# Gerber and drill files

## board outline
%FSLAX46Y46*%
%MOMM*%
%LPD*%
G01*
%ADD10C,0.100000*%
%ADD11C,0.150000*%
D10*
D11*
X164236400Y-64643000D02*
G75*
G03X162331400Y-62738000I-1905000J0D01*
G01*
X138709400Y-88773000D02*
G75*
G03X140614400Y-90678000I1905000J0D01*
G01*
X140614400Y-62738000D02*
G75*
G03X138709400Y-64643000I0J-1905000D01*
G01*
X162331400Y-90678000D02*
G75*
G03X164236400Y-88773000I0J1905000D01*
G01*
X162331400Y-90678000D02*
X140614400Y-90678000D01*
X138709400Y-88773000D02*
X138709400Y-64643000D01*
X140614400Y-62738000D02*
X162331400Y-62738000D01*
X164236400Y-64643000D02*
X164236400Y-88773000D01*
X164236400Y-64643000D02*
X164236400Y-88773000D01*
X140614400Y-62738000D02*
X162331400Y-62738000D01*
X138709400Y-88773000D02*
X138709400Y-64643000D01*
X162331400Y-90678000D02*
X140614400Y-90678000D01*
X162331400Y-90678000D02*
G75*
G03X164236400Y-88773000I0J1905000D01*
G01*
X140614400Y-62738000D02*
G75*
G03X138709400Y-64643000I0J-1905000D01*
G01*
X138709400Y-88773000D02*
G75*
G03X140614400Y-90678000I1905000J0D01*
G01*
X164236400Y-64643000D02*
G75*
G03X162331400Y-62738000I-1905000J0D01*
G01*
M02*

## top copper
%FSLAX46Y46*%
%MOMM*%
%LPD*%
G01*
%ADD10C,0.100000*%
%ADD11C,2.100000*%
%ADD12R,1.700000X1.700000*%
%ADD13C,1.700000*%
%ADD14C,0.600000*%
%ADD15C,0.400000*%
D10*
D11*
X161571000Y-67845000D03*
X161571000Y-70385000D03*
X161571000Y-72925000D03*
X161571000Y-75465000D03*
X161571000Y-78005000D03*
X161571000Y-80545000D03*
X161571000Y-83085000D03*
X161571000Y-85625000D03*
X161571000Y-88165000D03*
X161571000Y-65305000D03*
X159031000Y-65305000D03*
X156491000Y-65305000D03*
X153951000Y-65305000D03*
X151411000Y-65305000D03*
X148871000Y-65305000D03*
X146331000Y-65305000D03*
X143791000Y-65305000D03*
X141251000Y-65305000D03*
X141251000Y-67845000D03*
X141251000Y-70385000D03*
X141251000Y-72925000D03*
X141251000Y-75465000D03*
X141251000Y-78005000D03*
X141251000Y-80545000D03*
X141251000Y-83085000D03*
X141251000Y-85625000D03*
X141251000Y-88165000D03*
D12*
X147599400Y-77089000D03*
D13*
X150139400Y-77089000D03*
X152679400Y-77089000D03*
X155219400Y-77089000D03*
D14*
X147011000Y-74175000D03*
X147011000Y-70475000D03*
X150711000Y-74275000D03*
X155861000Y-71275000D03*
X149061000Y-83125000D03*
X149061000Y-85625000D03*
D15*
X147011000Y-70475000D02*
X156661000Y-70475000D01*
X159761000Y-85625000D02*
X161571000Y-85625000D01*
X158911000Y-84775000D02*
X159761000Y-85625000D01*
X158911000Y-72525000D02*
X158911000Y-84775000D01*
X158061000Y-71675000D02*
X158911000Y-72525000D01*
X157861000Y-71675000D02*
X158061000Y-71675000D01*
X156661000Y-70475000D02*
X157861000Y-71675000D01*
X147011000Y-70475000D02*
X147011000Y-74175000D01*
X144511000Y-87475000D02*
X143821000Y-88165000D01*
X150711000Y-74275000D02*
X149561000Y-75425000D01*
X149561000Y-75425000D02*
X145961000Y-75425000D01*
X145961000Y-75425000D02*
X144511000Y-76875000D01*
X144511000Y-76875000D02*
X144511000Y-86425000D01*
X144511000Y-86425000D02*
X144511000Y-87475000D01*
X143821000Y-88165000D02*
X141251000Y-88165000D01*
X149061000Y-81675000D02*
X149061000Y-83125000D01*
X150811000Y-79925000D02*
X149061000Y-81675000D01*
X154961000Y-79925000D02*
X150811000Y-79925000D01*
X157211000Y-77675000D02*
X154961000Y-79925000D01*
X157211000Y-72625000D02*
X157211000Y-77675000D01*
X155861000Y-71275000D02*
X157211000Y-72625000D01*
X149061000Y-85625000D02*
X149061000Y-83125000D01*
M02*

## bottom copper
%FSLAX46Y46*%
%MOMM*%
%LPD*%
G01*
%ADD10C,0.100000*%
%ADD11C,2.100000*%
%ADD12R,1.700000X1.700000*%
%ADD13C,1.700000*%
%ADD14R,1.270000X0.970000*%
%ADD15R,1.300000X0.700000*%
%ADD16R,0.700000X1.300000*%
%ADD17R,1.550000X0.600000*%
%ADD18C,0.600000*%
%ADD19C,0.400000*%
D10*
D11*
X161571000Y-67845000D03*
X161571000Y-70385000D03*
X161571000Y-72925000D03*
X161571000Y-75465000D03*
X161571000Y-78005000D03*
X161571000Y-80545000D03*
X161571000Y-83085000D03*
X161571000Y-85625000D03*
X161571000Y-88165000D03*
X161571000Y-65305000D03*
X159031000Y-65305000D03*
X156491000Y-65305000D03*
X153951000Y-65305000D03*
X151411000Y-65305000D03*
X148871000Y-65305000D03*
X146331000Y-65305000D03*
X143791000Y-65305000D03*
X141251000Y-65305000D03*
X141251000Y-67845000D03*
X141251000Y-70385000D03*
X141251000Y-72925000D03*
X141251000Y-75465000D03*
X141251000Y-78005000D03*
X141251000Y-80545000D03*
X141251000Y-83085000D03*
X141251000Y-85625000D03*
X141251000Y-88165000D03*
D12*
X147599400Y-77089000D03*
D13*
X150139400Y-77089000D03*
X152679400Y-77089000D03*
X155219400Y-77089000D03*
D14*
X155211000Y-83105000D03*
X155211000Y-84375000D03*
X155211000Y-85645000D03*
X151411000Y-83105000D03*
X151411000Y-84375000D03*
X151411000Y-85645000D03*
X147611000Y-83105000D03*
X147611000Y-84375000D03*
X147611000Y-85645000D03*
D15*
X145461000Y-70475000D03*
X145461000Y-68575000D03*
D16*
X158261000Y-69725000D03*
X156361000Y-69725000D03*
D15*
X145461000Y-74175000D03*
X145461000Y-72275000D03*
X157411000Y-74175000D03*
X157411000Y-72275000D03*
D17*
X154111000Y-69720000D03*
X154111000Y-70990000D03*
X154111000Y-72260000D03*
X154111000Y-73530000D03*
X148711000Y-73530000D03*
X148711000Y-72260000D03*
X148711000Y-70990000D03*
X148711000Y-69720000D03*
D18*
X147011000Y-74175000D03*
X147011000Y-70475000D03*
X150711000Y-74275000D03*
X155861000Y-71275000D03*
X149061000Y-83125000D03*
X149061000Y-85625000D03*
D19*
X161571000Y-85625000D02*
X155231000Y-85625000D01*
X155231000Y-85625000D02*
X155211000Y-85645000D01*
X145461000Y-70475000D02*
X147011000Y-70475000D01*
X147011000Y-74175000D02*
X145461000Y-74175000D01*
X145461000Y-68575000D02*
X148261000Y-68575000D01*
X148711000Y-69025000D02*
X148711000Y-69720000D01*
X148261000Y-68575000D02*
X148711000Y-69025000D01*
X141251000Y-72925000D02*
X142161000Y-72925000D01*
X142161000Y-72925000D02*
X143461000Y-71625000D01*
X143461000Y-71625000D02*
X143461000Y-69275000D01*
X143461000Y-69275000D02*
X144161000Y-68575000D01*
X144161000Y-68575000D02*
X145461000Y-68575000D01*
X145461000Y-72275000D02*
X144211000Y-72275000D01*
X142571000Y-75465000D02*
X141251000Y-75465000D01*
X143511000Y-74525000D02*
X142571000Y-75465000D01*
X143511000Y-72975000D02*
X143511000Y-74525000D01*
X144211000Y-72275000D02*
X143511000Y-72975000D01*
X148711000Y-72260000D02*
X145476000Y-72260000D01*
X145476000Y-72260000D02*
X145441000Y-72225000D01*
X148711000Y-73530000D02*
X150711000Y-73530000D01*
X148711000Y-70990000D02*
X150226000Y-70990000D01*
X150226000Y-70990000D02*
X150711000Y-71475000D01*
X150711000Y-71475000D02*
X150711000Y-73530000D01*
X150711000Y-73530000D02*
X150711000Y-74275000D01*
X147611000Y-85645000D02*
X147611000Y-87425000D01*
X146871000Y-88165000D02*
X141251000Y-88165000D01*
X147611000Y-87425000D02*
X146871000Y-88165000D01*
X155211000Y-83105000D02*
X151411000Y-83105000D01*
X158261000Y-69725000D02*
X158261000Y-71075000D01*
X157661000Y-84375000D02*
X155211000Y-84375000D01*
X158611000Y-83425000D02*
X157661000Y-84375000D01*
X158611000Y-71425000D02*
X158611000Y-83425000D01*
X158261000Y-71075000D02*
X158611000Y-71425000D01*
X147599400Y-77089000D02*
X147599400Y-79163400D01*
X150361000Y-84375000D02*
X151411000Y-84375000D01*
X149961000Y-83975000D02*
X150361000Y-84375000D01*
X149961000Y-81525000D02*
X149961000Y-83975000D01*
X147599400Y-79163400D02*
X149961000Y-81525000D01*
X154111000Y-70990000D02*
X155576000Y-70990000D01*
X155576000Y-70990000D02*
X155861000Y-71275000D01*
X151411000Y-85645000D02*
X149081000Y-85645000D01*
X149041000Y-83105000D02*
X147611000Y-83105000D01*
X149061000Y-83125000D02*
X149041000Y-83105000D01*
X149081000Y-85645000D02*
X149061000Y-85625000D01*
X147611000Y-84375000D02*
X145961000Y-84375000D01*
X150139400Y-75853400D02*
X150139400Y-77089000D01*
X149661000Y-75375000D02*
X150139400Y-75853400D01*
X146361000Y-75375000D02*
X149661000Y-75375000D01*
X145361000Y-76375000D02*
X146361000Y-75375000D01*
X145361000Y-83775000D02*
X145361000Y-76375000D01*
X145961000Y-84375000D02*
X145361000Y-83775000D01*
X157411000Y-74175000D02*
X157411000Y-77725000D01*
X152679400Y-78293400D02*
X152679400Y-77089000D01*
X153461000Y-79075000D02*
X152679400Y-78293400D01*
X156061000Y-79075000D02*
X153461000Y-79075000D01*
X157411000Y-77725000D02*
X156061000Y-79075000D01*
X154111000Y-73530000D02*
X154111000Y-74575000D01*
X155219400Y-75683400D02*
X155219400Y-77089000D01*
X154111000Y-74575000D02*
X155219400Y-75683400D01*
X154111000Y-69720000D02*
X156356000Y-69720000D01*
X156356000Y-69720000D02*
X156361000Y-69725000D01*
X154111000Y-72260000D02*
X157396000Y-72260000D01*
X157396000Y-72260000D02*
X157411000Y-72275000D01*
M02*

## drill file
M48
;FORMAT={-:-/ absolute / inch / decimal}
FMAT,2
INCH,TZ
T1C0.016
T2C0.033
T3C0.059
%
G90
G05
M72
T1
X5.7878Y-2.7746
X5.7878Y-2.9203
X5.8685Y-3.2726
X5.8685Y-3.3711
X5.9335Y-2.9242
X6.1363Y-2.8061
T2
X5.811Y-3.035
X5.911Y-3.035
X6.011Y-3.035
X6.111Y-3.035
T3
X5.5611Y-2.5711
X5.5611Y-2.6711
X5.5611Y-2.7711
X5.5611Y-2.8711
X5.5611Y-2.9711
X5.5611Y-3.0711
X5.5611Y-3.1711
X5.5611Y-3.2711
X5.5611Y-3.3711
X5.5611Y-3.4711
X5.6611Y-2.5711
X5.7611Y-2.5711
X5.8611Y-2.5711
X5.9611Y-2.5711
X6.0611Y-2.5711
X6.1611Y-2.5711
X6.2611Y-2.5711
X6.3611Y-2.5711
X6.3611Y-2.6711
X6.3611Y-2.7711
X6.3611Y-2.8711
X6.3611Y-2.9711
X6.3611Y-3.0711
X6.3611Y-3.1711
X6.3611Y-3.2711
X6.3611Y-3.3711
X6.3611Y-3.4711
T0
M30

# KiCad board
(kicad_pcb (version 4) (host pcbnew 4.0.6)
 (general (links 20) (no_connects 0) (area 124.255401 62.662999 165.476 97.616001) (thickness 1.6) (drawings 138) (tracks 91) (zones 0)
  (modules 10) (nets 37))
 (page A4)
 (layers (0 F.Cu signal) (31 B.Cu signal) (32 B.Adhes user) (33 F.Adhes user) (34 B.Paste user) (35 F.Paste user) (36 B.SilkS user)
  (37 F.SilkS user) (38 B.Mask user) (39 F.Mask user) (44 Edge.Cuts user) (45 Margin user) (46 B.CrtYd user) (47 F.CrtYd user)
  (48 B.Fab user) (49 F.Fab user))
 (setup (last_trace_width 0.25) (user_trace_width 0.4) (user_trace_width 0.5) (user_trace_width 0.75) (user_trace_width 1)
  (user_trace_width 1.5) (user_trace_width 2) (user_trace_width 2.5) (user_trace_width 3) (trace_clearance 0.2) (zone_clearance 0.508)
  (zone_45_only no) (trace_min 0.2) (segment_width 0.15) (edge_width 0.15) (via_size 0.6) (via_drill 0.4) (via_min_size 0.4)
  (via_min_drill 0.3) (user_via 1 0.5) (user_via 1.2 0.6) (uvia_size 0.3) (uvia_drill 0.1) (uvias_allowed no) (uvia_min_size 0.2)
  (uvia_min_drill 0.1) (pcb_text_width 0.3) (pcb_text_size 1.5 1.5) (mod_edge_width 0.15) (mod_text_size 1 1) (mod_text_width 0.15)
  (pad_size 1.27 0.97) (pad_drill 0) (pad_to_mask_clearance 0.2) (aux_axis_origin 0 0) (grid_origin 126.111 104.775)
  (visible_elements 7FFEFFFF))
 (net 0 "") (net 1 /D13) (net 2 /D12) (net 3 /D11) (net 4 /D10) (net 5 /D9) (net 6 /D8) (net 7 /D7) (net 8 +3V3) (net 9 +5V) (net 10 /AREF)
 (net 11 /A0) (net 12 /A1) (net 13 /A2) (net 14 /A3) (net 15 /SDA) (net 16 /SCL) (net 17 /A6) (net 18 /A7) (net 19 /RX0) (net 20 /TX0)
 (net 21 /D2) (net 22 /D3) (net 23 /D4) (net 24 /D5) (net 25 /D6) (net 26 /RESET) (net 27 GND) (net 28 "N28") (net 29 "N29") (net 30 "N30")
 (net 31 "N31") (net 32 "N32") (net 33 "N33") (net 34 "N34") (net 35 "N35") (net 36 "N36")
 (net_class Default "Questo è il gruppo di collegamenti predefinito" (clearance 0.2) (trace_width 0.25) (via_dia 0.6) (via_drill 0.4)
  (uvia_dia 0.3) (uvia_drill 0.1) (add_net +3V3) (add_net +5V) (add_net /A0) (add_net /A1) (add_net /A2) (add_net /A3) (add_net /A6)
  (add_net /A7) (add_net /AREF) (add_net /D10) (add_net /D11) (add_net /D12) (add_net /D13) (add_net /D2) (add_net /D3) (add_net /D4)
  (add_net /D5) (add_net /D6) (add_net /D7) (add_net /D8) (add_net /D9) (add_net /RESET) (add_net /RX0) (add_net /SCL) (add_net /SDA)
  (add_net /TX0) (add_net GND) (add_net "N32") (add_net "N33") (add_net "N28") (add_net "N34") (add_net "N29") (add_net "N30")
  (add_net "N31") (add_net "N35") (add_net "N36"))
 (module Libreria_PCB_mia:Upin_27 (layer B.Cu) (at 161.571 88.165 180)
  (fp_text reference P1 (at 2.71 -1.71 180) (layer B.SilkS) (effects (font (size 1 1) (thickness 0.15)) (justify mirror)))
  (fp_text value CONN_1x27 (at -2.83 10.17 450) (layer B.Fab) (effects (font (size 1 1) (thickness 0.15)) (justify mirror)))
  (pad 9 thru_hole circle (at 0 20.32 180) (size 2.1 2.1) (drill 1.5) (layers *.Cu *.Mask) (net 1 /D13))
  (pad 8 thru_hole circle (at 0 17.78 180) (size 2.1 2.1) (drill 1.5) (layers *.Cu *.Mask) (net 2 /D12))
  (pad 7 thru_hole circle (at 0 15.24 180) (size 2.1 2.1) (drill 1.5) (layers *.Cu *.Mask) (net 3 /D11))
  (pad 6 thru_hole circle (at 0 12.7 180) (size 2.1 2.1) (drill 1.5) (layers *.Cu *.Mask) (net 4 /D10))
  (pad 5 thru_hole circle (at 0 10.16 180) (size 2.1 2.1) (drill 1.5) (layers *.Cu *.Mask) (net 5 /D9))
  (pad 4 thru_hole circle (at 0 7.62 180) (size 2.1 2.1) (drill 1.5) (layers *.Cu *.Mask) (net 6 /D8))
  (pad 3 thru_hole circle (at 0 5.08 180) (size 2.1 2.1) (drill 1.5) (layers *.Cu *.Mask) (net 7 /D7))
  (pad 2 thru_hole circle (at 0 2.54 180) (size 2.1 2.1) (drill 1.5) (layers *.Cu *.Mask) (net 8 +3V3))
  (pad 1 thru_hole circle (at 0 0 180) (size 2.1 2.1) (drill 1.5) (layers *.Cu *.Mask) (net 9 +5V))
  (pad 10 thru_hole circle (at 0 22.86 180) (size 2.1 2.1) (drill 1.5) (layers *.Cu *.Mask) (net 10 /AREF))
  (pad 11 thru_hole circle (at 2.54 22.86 180) (size 2.1 2.1) (drill 1.5) (layers *.Cu *.Mask) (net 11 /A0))
  (pad 12 thru_hole circle (at 5.08 22.86 180) (size 2.1 2.1) (drill 1.5) (layers *.Cu *.Mask) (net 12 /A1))
  (pad 13 thru_hole circle (at 7.62 22.86 180) (size 2.1 2.1) (drill 1.5) (layers *.Cu *.Mask) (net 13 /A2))
  (pad 14 thru_hole circle (at 10.16 22.86 180) (size 2.1 2.1) (drill 1.5) (layers *.Cu *.Mask) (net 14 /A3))
  (pad 15 thru_hole circle (at 12.7 22.86 180) (size 2.1 2.1) (drill 1.5) (layers *.Cu *.Mask) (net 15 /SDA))
  (pad 16 thru_hole circle (at 15.24 22.86 180) (size 2.1 2.1) (drill 1.5) (layers *.Cu *.Mask) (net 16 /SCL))
  (pad 17 thru_hole circle (at 17.78 22.86 180) (size 2.1 2.1) (drill 1.5) (layers *.Cu *.Mask) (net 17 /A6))
  (pad 18 thru_hole circle (at 20.32 22.86 180) (size 2.1 2.1) (drill 1.5) (layers *.Cu *.Mask) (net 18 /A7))
  (pad 19 thru_hole circle (at 20.32 20.32 180) (size 2.1 2.1) (drill 1.5) (layers *.Cu *.Mask) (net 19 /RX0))
  (pad 20 thru_hole circle (at 20.32 17.78 180) (size 2.1 2.1) (drill 1.5) (layers *.Cu *.Mask) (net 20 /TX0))
  (pad 21 thru_hole circle (at 20.32 15.24 180) (size 2.1 2.1) (drill 1.5) (layers *.Cu *.Mask) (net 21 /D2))
  (pad 22 thru_hole circle (at 20.32 12.7 180) (size 2.1 2.1) (drill 1.5) (layers *.Cu *.Mask) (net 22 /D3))
  (pad 23 thru_hole circle (at 20.32 10.16 180) (size 2.1 2.1) (drill 1.5) (layers *.Cu *.Mask) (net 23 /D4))
  (pad 24 thru_hole circle (at 20.32 7.62 180) (size 2.1 2.1) (drill 1.5) (layers *.Cu *.Mask) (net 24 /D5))
  (pad 25 thru_hole circle (at 20.32 5.08 180) (size 2.1 2.1) (drill 1.5) (layers *.Cu *.Mask) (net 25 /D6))
  (pad 26 thru_hole circle (at 20.32 2.54 180) (size 2.1 2.1) (drill 1.5) (layers *.Cu *.Mask) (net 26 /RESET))
  (pad 27 thru_hole circle (at 20.32 0 180) (size 2.1 2.1) (drill 1.5) (layers *.Cu *.Mask) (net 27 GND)))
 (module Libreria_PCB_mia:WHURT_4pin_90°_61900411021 (layer F.Cu) (at 147.5994 77.089)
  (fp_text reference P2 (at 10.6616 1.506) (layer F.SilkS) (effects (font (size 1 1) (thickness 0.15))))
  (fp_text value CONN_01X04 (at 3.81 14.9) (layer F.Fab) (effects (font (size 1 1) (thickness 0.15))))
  (pad 1 thru_hole rect (at 0 0) (size 1.7 1.7) (drill 0.85) (layers *.Cu *.Mask) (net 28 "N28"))
  (pad 2 thru_hole circle (at 2.54 0) (size 1.7 1.7) (drill 0.85) (layers *.Cu *.Mask) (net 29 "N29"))
  (pad 3 thru_hole circle (at 5.08 0) (size 1.7 1.7) (drill 0.85) (layers *.Cu *.Mask) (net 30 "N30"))
  (pad 4 thru_hole circle (at 7.62 0) (size 1.7 1.7) (drill 0.85) (layers *.Cu *.Mask) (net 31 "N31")))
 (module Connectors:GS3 (layer B.Cu) (at 155.211 84.375 180)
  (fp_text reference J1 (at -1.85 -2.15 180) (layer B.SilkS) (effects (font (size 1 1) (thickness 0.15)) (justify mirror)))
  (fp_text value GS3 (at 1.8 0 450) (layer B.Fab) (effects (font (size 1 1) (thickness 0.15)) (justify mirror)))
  (pad 1 smd rect (at 0 1.27 180) (size 1.27 0.97) (layers B.Cu B.Paste B.Mask) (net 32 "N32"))
  (pad 2 smd rect (at 0 0 180) (size 1.27 0.97) (layers B.Cu B.Paste B.Mask) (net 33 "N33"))
  (pad 3 smd rect (at 0 -1.27 180) (size 1.27 0.97) (layers B.Cu B.Paste B.Mask) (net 8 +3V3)))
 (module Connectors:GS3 (layer B.Cu) (at 151.411 84.375 180)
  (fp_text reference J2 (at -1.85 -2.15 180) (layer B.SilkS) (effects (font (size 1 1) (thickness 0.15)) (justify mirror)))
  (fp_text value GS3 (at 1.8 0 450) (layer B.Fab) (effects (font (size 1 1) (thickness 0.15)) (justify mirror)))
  (pad 1 smd rect (at 0 1.27 180) (size 1.27 0.97) (layers B.Cu B.Paste B.Mask) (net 32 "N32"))
  (pad 2 smd rect (at 0 0 180) (size 1.27 0.97) (layers B.Cu B.Paste B.Mask) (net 28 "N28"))
  (pad 3 smd rect (at 0 -1.27 180) (size 1.27 0.97) (layers B.Cu B.Paste B.Mask) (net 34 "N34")))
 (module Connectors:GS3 (layer B.Cu) (at 147.611 84.375 180)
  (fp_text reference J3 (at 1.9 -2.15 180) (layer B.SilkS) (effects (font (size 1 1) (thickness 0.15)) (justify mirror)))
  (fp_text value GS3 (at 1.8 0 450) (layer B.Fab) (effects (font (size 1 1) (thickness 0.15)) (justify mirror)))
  (pad 1 smd rect (at 0 1.27 180) (size 1.27 0.97) (layers B.Cu B.Paste B.Mask) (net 34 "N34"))
  (pad 2 smd rect (at 0 0 180) (size 1.27 0.97) (layers B.Cu B.Paste B.Mask) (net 29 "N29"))
  (pad 3 smd rect (at 0 -1.27 180) (size 1.27 0.97) (layers B.Cu B.Paste B.Mask) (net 27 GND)))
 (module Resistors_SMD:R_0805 (layer B.Cu) (at 145.461 69.525 90)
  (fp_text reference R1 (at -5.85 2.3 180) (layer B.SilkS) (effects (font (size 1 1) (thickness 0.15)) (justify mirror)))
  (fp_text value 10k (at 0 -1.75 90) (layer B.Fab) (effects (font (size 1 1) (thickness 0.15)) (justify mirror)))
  (pad 1 smd rect (at -0.95 0 90) (size 0.7 1.3) (layers B.Cu B.Paste B.Mask) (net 8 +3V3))
  (pad 2 smd rect (at 0.95 0 90) (size 0.7 1.3) (layers B.Cu B.Paste B.Mask) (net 21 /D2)))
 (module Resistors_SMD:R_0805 (layer B.Cu) (at 157.311 69.725 180)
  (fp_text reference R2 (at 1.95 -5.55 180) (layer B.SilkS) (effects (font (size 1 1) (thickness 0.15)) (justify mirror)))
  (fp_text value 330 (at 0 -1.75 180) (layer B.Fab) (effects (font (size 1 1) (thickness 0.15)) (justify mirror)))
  (pad 1 smd rect (at -0.95 0 180) (size 0.7 1.3) (layers B.Cu B.Paste B.Mask) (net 33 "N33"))
  (pad 2 smd rect (at 0.95 0 180) (size 0.7 1.3) (layers B.Cu B.Paste B.Mask) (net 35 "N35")))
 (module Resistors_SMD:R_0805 (layer B.Cu) (at 145.461 73.225 90)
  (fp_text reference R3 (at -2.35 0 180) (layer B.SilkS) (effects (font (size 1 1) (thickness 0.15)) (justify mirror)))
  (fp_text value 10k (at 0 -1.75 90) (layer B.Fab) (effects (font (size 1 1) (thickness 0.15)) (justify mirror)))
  (pad 1 smd rect (at -0.95 0 90) (size 0.7 1.3) (layers B.Cu B.Paste B.Mask) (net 8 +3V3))
  (pad 2 smd rect (at 0.95 0 90) (size 0.7 1.3) (layers B.Cu B.Paste B.Mask) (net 22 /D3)))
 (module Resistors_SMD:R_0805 (layer B.Cu) (at 157.411 73.225 90)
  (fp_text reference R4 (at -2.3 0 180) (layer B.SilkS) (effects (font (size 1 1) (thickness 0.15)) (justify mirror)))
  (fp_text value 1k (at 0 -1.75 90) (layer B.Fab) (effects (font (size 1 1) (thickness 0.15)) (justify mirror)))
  (pad 1 smd rect (at -0.95 0 90) (size 0.7 1.3) (layers B.Cu B.Paste B.Mask) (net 30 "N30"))
  (pad 2 smd rect (at 0.95 0 90) (size 0.7 1.3) (layers B.Cu B.Paste B.Mask) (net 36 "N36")))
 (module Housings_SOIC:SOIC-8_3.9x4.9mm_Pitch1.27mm (layer B.Cu) (at 151.411 71.625 180)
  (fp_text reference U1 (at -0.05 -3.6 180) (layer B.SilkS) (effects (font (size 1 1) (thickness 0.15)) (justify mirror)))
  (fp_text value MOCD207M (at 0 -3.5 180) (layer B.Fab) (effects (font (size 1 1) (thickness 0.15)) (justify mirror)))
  (pad 1 smd rect (at -2.7 1.905 180) (size 1.55 0.6) (layers B.Cu B.Paste B.Mask) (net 35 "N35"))
  (pad 2 smd rect (at -2.7 0.635 180) (size 1.55 0.6) (layers B.Cu B.Paste B.Mask) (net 34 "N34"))
  (pad 3 smd rect (at -2.7 -0.635 180) (size 1.55 0.6) (layers B.Cu B.Paste B.Mask) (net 36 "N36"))
  (pad 4 smd rect (at -2.7 -1.905 180) (size 1.55 0.6) (layers B.Cu B.Paste B.Mask) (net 31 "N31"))
  (pad 5 smd rect (at 2.7 -1.905 180) (size 1.55 0.6) (layers B.Cu B.Paste B.Mask) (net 27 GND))
  (pad 6 smd rect (at 2.7 -0.635 180) (size 1.55 0.6) (layers B.Cu B.Paste B.Mask) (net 22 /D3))
  (pad 7 smd rect (at 2.7 0.635 180) (size 1.55 0.6) (layers B.Cu B.Paste B.Mask) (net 27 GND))
  (pad 8 smd rect (at 2.7 1.905 180) (size 1.55 0.6) (layers B.Cu B.Paste B.Mask) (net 21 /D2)))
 (gr_arc (start 162.3314 64.643) (end 162.3314 62.738) (angle 90) (layer Edge.Cuts) (width 0.15))
 (gr_arc (start 140.6144 88.773) (end 140.6144 90.678) (angle 90) (layer Edge.Cuts) (width 0.15))
 (gr_arc (start 140.6144 64.643) (end 138.7094 64.643) (angle 90) (layer Edge.Cuts) (width 0.15))
 (gr_arc (start 162.3314 88.773) (end 164.2364 88.773) (angle 90) (layer Edge.Cuts) (width 0.15))
 (gr_line (start 162.3314 90.678) (end 140.6144 90.678) (angle 90) (layer Edge.Cuts) (width 0.15))
 (gr_line (start 138.7094 88.773) (end 138.7094 64.643) (angle 90) (layer Edge.Cuts) (width 0.15))
 (gr_line (start 140.6144 62.738) (end 162.3314 62.738) (angle 90) (layer Edge.Cuts) (width 0.15))
 (gr_line (start 164.2364 64.643) (end 164.2364 88.773) (angle 90) (layer Edge.Cuts) (width 0.15))
 (gr_line (start 164.2364 64.643) (end 164.2364 88.773) (angle 90) (layer Edge.Cuts) (width 0.15))
 (gr_line (start 140.6144 62.738) (end 162.3314 62.738) (angle 90) (layer Edge.Cuts) (width 0.15))
 (gr_line (start 138.7094 88.773) (end 138.7094 64.643) (angle 90) (layer Edge.Cuts) (width 0.15))
 (gr_line (start 162.3314 90.678) (end 140.6144 90.678) (angle 90) (layer Edge.Cuts) (width 0.15))
 (gr_arc (start 162.3314 88.773) (end 164.2364 88.773) (angle 90) (layer Edge.Cuts) (width 0.15))
 (gr_arc (start 140.6144 64.643) (end 138.7094 64.643) (angle 90) (layer Edge.Cuts) (width 0.15))
 (gr_arc (start 140.6144 88.773) (end 140.6144 90.678) (angle 90) (layer Edge.Cuts) (width 0.15))
 (gr_arc (start 162.3314 64.643) (end 162.3314 62.738) (angle 90) (layer Edge.Cuts) (width 0.15))
 (segment (start 147.011 70.475) (end 156.661 70.475) (width 0.4) (layer F.Cu) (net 8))
 (segment (start 159.761 85.625) (end 161.571 85.625) (width 0.4) (layer F.Cu) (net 8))
 (segment (start 158.911 84.775) (end 159.761 85.625) (width 0.4) (layer F.Cu) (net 8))
 (segment (start 158.911 72.525) (end 158.911 84.775) (width 0.4) (layer F.Cu) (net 8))
 (segment (start 158.061 71.675) (end 158.911 72.525) (width 0.4) (layer F.Cu) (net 8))
 (segment (start 157.861 71.675) (end 158.061 71.675) (width 0.4) (layer F.Cu) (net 8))
 (segment (start 156.661 70.475) (end 157.861 71.675) (width 0.4) (layer F.Cu) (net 8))
 (segment (start 161.571 85.625) (end 155.231 85.625) (width 0.4) (layer B.Cu) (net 8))
 (segment (start 155.231 85.625) (end 155.211 85.645) (width 0.4) (layer B.Cu) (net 8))
 (segment (start 145.461 70.475) (end 147.011 70.475) (width 0.4) (layer B.Cu) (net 8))
 (segment (start 147.011 74.175) (end 145.461 74.175) (width 0.4) (layer B.Cu) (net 8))
 (via (at 147.011 74.175) (size 0.6) (drill 0.4) (layers F.Cu B.Cu) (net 8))
 (segment (start 147.011 70.475) (end 147.011 74.175) (width 0.4) (layer F.Cu) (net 8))
 (via (at 147.011 70.475) (size 0.6) (drill 0.4) (layers F.Cu B.Cu) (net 8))
 (segment (start 145.461 68.575) (end 148.261 68.575) (width 0.4) (layer B.Cu) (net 21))
 (segment (start 148.711 69.025) (end 148.711 69.72) (width 0.4) (layer B.Cu) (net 21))
 (segment (start 148.261 68.575) (end 148.711 69.025) (width 0.4) (layer B.Cu) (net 21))
 (segment (start 141.251 72.925) (end 142.161 72.925) (width 0.4) (layer B.Cu) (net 21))
 (segment (start 142.161 72.925) (end 143.461 71.625) (width 0.4) (layer B.Cu) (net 21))
 (segment (start 143.461 71.625) (end 143.461 69.275) (width 0.4) (layer B.Cu) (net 21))
 (segment (start 143.461 69.275) (end 144.161 68.575) (width 0.4) (layer B.Cu) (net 21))
 (segment (start 144.161 68.575) (end 145.461 68.575) (width 0.4) (layer B.Cu) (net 21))
 (segment (start 145.461 72.275) (end 144.211 72.275) (width 0.4) (layer B.Cu) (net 22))
 (segment (start 142.571 75.465) (end 141.251 75.465) (width 0.4) (layer B.Cu) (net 22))
 (segment (start 143.511 74.525) (end 142.571 75.465) (width 0.4) (layer B.Cu) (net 22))
 (segment (start 143.511 72.975) (end 143.511 74.525) (width 0.4) (layer B.Cu) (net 22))
 (segment (start 144.211 72.275) (end 143.511 72.975) (width 0.4) (layer B.Cu) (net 22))
 (segment (start 148.711 72.26) (end 145.476 72.26) (width 0.4) (layer B.Cu) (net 22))
 (segment (start 145.476 72.26) (end 145.441 72.225) (width 0.4) (layer B.Cu) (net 22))
 (segment (start 148.711 73.53) (end 150.711 73.53) (width 0.4) (layer B.Cu) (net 27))
 (segment (start 144.511 87.475) (end 143.821 88.165) (width 0.4) (layer F.Cu) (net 27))
 (segment (start 148.711 70.99) (end 150.226 70.99) (width 0.4) (layer B.Cu) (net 27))
 (segment (start 150.226 70.99) (end 150.711 71.475) (width 0.4) (layer B.Cu) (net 27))
 (segment (start 150.711 71.475) (end 150.711 73.53) (width 0.4) (layer B.Cu) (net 27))
 (segment (start 150.711 73.53) (end 150.711 74.275) (width 0.4) (layer B.Cu) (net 27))
 (via (at 150.711 74.275) (size 0.6) (drill 0.4) (layers F.Cu B.Cu) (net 27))
 (segment (start 150.711 74.275) (end 149.561 75.425) (width 0.4) (layer F.Cu) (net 27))
 (segment (start 149.561 75.425) (end 145.961 75.425) (width 0.4) (layer F.Cu) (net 27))
 (segment (start 145.961 75.425) (end 144.511 76.875) (width 0.4) (layer F.Cu) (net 27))
 (segment (start 144.511 76.875) (end 144.511 86.425) (width 0.4) (layer F.Cu) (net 27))
 (segment (start 144.511 86.425) (end 144.511 87.475) (width 0.4) (layer F.Cu) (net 27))
 (segment (start 143.821 88.165) (end 141.251 88.165) (width 0.4) (layer F.Cu) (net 27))
 (segment (start 147.611 85.645) (end 147.611 87.425) (width 0.4) (layer B.Cu) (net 27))
 (segment (start 146.871 88.165) (end 141.251 88.165) (width 0.4) (layer B.Cu) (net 27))
 (segment (start 147.611 87.425) (end 146.871 88.165) (width 0.4) (layer B.Cu) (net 27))
 (segment (start 155.211 83.105) (end 151.411 83.105) (width 0.4) (layer B.Cu) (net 32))
 (segment (start 158.261 69.725) (end 158.261 71.075) (width 0.4) (layer B.Cu) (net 33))
 (segment (start 157.661 84.375) (end 155.211 84.375) (width 0.4) (layer B.Cu) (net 33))
 (segment (start 158.611 83.425) (end 157.661 84.375) (width 0.4) (layer B.Cu) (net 33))
 (segment (start 158.611 71.425) (end 158.611 83.425) (width 0.4) (layer B.Cu) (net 33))
 (segment (start 158.261 71.075) (end 158.611 71.425) (width 0.4) (layer B.Cu) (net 33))
 (segment (start 147.5994 77.089) (end 147.5994 79.1634) (width 0.4) (layer B.Cu) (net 28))
 (segment (start 150.361 84.375) (end 151.411 84.375) (width 0.4) (layer B.Cu) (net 28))
 (segment (start 149.961 83.975) (end 150.361 84.375) (width 0.4) (layer B.Cu) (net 28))
 (segment (start 149.961 81.525) (end 149.961 83.975) (width 0.4) (layer B.Cu) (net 28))
 (segment (start 147.5994 79.1634) (end 149.961 81.525) (width 0.4) (layer B.Cu) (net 28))
 (segment (start 154.111 70.99) (end 155.576 70.99) (width 0.4) (layer B.Cu) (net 34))
 (segment (start 149.061 81.675) (end 149.061 83.125) (width 0.4) (layer F.Cu) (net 34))
 (segment (start 150.811 79.925) (end 149.061 81.675) (width 0.4) (layer F.Cu) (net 34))
 (segment (start 154.961 79.925) (end 150.811 79.925) (width 0.4) (layer F.Cu) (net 34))
 (segment (start 157.211 77.675) (end 154.961 79.925) (width 0.4) (layer F.Cu) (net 34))
 (segment (start 157.211 72.625) (end 157.211 77.675) (width 0.4) (layer F.Cu) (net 34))
 (segment (start 155.861 71.275) (end 157.211 72.625) (width 0.4) (layer F.Cu) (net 34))
 (via (at 155.861 71.275) (size 0.6) (drill 0.4) (layers F.Cu B.Cu) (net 34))
 (segment (start 155.576 70.99) (end 155.861 71.275) (width 0.4) (layer B.Cu) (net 34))
 (segment (start 151.411 85.645) (end 149.081 85.645) (width 0.4) (layer B.Cu) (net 34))
 (segment (start 149.041 83.105) (end 147.611 83.105) (width 0.4) (layer B.Cu) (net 34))
 (segment (start 149.061 83.125) (end 149.041 83.105) (width 0.4) (layer B.Cu) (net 34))
 (via (at 149.061 83.125) (size 0.6) (drill 0.4) (layers F.Cu B.Cu) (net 34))
 (segment (start 149.061 85.625) (end 149.061 83.125) (width 0.4) (layer F.Cu) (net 34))
 (via (at 149.061 85.625) (size 0.6) (drill 0.4) (layers F.Cu B.Cu) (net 34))
 (segment (start 149.081 85.645) (end 149.061 85.625) (width 0.4) (layer B.Cu) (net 34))
 (segment (start 147.611 84.375) (end 145.961 84.375) (width 0.4) (layer B.Cu) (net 29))
 (segment (start 150.1394 75.8534) (end 150.1394 77.089) (width 0.4) (layer B.Cu) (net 29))
 (segment (start 149.661 75.375) (end 150.1394 75.8534) (width 0.4) (layer B.Cu) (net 29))
 (segment (start 146.361 75.375) (end 149.661 75.375) (width 0.4) (layer B.Cu) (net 29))
 (segment (start 145.361 76.375) (end 146.361 75.375) (width 0.4) (layer B.Cu) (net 29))
 (segment (start 145.361 83.775) (end 145.361 76.375) (width 0.4) (layer B.Cu) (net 29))
 (segment (start 145.961 84.375) (end 145.361 83.775) (width 0.4) (layer B.Cu) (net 29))
 (segment (start 157.411 74.175) (end 157.411 77.725) (width 0.4) (layer B.Cu) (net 30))
 (segment (start 152.6794 78.2934) (end 152.6794 77.089) (width 0.4) (layer B.Cu) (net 30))
 (segment (start 153.461 79.075) (end 152.6794 78.2934) (width 0.4) (layer B.Cu) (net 30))
 (segment (start 156.061 79.075) (end 153.461 79.075) (width 0.4) (layer B.Cu) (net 30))
 (segment (start 157.411 77.725) (end 156.061 79.075) (width 0.4) (layer B.Cu) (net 30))
 (segment (start 154.111 73.53) (end 154.111 74.575) (width 0.4) (layer B.Cu) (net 31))
 (segment (start 155.2194 75.6834) (end 155.2194 77.089) (width 0.4) (layer B.Cu) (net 31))
 (segment (start 154.111 74.575) (end 155.2194 75.6834) (width 0.4) (layer B.Cu) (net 31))
 (segment (start 154.111 69.72) (end 156.356 69.72) (width 0.4) (layer B.Cu) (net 35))
 (segment (start 156.356 69.72) (end 156.361 69.725) (width 0.4) (layer B.Cu) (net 35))
 (segment (start 154.111 72.26) (end 157.396 72.26) (width 0.4) (layer B.Cu) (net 36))
 (segment (start 157.396 72.26) (end 157.411 72.275) (width 0.4) (layer B.Cu) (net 36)))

